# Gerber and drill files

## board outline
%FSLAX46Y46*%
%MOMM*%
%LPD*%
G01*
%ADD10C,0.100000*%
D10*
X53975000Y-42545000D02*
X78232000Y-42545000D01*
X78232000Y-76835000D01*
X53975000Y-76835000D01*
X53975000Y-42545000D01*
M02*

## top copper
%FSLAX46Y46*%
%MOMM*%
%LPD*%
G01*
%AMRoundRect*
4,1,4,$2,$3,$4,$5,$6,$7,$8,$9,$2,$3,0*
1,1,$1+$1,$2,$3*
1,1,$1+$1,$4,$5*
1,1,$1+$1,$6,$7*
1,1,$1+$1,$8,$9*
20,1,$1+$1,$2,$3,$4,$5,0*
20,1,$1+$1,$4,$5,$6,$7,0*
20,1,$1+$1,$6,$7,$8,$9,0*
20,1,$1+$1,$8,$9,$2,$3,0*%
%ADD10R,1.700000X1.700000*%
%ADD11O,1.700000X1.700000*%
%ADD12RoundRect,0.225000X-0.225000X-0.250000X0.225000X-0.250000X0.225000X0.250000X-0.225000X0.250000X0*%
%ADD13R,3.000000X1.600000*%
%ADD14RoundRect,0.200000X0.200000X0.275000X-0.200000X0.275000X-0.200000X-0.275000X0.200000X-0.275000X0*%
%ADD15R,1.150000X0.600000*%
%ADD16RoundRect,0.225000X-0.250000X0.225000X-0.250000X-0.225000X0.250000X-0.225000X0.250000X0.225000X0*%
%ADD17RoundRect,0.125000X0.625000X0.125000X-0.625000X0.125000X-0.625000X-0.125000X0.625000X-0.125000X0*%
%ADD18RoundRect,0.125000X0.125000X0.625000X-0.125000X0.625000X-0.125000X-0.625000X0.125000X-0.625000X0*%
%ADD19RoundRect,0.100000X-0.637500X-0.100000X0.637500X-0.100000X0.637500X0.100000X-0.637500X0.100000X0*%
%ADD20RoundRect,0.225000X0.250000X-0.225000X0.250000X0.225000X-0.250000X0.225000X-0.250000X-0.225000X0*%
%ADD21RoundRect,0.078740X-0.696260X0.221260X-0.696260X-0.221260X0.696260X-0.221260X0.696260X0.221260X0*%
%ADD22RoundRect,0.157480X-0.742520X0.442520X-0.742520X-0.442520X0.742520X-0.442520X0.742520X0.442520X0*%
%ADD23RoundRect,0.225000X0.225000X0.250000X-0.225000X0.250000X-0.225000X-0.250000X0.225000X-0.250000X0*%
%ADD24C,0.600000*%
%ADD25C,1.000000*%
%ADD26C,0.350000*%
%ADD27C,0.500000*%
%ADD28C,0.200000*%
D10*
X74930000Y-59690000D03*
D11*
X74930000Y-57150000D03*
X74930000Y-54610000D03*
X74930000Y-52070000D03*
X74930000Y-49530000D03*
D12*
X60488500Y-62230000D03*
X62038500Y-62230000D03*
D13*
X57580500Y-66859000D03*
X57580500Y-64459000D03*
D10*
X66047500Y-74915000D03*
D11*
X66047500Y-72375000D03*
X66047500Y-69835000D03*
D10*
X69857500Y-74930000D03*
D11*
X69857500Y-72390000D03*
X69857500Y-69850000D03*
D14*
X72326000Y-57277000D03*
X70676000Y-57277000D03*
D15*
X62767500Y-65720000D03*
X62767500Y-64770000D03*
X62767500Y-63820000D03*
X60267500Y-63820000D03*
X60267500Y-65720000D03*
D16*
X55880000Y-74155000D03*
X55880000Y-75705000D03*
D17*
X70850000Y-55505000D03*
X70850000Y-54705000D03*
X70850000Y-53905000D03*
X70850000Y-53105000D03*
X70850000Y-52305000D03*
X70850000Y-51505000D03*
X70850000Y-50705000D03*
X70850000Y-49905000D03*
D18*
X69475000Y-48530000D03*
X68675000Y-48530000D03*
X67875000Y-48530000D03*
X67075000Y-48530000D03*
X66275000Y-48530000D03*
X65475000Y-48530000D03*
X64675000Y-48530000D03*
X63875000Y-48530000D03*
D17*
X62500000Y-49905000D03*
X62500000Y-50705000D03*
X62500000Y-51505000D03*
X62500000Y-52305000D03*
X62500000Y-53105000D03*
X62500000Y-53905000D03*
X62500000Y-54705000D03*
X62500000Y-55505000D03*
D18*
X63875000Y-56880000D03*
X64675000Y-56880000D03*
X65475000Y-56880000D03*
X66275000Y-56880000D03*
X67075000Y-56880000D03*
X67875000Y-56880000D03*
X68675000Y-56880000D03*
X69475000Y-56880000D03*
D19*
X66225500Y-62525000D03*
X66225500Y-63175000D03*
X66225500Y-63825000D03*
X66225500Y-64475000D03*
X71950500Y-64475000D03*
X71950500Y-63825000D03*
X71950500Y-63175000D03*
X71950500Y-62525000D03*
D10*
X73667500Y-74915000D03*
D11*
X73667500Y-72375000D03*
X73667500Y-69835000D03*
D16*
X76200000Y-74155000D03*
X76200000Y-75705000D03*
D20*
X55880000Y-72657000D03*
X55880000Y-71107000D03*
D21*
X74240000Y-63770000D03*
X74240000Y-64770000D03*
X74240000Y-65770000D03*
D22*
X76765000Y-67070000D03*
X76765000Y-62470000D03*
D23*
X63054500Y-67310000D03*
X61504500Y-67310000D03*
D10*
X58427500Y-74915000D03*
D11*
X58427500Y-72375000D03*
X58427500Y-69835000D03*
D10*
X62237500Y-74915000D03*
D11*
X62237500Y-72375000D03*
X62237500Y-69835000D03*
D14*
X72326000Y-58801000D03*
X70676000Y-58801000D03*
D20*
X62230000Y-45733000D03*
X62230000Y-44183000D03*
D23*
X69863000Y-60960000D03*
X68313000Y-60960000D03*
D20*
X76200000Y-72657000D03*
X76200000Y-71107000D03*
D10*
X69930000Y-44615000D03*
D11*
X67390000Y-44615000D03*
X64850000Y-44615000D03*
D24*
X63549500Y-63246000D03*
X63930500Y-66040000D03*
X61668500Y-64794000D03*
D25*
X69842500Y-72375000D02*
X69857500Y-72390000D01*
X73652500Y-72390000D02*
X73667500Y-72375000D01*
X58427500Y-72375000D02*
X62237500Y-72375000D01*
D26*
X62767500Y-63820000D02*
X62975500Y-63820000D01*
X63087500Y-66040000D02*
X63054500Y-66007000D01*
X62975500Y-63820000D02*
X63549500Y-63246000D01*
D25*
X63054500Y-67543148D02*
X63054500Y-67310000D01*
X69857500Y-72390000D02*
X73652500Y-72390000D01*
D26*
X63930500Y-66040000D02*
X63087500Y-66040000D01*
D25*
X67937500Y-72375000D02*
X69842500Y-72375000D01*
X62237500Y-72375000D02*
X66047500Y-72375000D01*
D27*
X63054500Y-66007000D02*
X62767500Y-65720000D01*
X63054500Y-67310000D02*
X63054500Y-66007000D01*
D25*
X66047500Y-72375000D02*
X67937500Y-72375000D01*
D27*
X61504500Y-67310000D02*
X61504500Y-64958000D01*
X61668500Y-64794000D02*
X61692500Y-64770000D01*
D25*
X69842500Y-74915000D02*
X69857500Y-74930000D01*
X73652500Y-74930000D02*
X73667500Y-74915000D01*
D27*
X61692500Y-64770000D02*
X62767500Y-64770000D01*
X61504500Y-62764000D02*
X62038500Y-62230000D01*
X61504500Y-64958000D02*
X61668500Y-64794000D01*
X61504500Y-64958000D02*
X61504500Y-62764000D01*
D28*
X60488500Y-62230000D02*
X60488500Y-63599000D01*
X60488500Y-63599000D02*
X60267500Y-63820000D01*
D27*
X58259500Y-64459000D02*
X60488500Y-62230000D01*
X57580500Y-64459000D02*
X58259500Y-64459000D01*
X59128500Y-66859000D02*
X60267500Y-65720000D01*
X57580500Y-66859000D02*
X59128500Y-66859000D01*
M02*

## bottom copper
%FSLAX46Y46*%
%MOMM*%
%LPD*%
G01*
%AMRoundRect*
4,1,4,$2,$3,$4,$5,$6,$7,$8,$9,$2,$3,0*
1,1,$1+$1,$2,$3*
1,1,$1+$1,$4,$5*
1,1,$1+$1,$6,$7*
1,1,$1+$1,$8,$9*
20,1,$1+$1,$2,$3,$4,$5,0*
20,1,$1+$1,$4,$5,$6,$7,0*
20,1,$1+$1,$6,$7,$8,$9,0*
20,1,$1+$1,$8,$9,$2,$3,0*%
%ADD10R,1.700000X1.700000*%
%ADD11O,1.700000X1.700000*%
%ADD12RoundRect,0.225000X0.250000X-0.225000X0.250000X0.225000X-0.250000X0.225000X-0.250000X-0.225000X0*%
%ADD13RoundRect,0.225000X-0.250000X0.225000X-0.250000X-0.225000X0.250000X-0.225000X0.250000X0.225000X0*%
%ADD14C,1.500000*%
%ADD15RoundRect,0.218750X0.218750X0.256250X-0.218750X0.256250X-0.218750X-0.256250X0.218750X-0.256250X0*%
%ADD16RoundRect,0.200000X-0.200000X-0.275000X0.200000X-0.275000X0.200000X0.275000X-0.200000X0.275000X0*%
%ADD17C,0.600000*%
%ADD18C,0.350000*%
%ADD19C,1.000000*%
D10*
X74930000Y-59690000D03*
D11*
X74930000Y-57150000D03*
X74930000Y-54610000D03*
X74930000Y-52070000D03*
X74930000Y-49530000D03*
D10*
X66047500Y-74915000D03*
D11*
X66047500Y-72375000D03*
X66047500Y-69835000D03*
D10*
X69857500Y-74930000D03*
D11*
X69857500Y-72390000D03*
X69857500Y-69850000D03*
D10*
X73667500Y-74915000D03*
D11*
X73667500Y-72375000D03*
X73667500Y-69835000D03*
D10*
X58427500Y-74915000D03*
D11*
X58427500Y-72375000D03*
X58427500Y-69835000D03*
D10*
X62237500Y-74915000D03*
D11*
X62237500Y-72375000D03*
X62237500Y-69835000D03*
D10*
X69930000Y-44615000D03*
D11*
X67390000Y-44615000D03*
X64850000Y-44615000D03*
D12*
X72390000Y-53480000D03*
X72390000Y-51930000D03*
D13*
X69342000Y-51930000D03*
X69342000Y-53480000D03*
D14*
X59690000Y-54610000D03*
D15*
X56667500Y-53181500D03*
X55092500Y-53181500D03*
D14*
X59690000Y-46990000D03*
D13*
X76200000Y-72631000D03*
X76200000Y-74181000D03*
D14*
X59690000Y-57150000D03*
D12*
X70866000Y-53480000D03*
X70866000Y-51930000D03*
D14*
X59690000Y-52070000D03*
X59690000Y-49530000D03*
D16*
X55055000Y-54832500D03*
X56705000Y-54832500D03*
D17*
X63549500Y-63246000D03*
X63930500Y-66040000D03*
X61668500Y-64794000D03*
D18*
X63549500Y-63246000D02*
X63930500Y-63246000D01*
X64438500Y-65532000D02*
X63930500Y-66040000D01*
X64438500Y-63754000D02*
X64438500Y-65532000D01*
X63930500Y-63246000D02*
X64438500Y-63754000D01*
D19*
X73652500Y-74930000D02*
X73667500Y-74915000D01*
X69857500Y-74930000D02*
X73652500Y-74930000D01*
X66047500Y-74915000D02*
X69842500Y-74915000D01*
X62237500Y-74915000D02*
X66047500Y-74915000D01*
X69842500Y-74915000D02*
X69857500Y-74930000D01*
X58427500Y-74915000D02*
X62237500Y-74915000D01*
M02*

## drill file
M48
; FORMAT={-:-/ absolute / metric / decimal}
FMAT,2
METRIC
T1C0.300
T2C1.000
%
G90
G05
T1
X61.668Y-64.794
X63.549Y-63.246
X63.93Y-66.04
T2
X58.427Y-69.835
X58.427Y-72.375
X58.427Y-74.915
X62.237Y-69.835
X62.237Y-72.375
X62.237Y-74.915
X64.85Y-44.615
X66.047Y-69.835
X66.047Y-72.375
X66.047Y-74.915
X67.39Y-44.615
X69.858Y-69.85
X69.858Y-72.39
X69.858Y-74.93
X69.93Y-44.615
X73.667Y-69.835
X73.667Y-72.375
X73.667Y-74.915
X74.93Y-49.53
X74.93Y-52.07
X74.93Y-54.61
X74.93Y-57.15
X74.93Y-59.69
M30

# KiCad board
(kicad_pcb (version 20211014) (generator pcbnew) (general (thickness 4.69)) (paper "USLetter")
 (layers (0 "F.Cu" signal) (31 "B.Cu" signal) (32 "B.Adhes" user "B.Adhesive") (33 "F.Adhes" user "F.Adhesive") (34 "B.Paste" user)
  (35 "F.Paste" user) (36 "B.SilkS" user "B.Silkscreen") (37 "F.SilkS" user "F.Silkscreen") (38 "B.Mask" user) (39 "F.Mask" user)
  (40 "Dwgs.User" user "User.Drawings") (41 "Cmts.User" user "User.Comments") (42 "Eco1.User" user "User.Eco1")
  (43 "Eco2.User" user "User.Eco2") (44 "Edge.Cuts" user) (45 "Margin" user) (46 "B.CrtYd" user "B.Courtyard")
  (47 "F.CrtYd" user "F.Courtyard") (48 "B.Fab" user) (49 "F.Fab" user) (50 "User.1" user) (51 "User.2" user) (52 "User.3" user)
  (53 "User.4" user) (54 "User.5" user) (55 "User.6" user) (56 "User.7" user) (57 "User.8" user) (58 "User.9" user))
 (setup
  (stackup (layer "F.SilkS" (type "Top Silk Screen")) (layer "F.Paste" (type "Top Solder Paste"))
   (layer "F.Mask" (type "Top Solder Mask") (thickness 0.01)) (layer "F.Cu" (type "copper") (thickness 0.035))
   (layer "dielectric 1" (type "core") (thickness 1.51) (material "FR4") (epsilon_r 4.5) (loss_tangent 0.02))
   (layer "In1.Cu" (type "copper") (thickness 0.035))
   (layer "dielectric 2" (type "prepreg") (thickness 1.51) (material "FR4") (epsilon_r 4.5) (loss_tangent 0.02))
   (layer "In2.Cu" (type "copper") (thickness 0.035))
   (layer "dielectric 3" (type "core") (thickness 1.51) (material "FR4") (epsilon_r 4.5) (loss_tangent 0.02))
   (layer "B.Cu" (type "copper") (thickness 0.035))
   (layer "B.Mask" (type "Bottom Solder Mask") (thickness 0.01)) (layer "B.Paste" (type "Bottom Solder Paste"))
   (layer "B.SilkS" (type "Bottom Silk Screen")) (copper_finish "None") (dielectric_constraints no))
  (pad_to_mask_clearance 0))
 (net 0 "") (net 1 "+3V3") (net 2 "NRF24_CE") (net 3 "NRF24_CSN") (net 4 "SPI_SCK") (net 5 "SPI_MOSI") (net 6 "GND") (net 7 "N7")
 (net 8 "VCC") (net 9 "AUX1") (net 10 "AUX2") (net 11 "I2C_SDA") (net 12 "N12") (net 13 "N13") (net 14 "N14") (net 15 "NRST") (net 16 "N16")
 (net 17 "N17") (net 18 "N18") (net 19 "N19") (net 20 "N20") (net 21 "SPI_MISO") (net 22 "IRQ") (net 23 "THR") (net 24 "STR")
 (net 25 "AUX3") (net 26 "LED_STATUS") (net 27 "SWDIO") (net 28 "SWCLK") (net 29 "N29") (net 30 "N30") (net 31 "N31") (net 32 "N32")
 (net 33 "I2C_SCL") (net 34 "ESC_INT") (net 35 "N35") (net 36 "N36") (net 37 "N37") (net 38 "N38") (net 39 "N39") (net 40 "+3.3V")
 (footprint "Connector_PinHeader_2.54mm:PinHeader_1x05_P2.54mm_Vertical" (layer "F.Cu") (at 74.93 59.69 180)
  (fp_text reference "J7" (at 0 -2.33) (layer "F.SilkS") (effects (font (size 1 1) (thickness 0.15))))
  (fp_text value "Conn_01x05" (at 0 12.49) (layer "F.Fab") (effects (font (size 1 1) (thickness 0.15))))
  (pad "1" thru_hole rect (at 0 0 180) (size 1.7 1.7) (drill 1) (layers *.Cu *.Mask) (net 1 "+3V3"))
  (pad "2" thru_hole oval (at 0 2.54 180) (size 1.7 1.7) (drill 1) (layers *.Cu *.Mask) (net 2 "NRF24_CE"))
  (pad "3" thru_hole oval (at 0 5.08 180) (size 1.7 1.7) (drill 1) (layers *.Cu *.Mask) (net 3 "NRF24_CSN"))
  (pad "4" thru_hole oval (at 0 7.62 180) (size 1.7 1.7) (drill 1) (layers *.Cu *.Mask) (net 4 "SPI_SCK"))
  (pad "5" thru_hole oval (at 0 10.16 180) (size 1.7 1.7) (drill 1) (layers *.Cu *.Mask) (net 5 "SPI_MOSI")))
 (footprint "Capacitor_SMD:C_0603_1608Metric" (layer "F.Cu") (at 61.2635 62.23)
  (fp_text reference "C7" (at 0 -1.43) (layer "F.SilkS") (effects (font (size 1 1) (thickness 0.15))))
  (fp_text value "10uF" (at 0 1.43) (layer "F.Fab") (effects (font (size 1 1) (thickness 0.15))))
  (pad "1" smd roundrect (at -0.775 0) (size 0.9 0.95) (layers "F.Cu" "F.Paste" "F.Mask") (roundrect_rratio 0.25) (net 1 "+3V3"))
  (pad "2" smd roundrect (at 0.775 0) (size 0.9 0.95) (layers "F.Cu" "F.Paste" "F.Mask") (roundrect_rratio 0.25) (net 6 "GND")))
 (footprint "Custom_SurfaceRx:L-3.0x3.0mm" (layer "F.Cu") (at 57.5805 65.659 90)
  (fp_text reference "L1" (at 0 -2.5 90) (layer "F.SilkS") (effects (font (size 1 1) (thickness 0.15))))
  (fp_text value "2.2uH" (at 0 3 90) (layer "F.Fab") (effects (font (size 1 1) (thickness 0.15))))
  (pad "1" smd rect (at -1.2 0 90) (size 1.6 3) (layers "F.Cu" "F.Paste" "F.Mask") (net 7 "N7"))
  (pad "2" smd rect (at 1.2 0 90) (size 1.6 3) (layers "F.Cu" "F.Paste" "F.Mask") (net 1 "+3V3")))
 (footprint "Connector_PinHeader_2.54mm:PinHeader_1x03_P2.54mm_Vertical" (layer "F.Cu") (at 66.0475 74.915 180)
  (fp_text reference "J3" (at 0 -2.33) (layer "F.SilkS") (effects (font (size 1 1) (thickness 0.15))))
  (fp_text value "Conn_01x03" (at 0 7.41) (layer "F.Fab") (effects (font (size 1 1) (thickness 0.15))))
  (pad "1" thru_hole rect (at 0 0 180) (size 1.7 1.7) (drill 1) (layers *.Cu *.Mask) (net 6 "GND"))
  (pad "2" thru_hole oval (at 0 2.54 180) (size 1.7 1.7) (drill 1) (layers *.Cu *.Mask) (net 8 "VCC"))
  (pad "3" thru_hole oval (at 0 5.08 180) (size 1.7 1.7) (drill 1) (layers *.Cu *.Mask) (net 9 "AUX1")))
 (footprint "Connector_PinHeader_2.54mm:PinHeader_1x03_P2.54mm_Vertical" (layer "F.Cu") (at 69.8575 74.93 180)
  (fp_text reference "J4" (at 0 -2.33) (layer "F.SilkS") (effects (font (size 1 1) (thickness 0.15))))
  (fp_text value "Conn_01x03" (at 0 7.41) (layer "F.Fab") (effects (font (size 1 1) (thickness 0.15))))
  (pad "1" thru_hole rect (at 0 0 180) (size 1.7 1.7) (drill 1) (layers *.Cu *.Mask) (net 6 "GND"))
  (pad "2" thru_hole oval (at 0 2.54 180) (size 1.7 1.7) (drill 1) (layers *.Cu *.Mask) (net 8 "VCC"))
  (pad "3" thru_hole oval (at 0 5.08 180) (size 1.7 1.7) (drill 1) (layers *.Cu *.Mask) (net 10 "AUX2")))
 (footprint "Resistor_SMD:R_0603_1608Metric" (layer "F.Cu") (at 71.501 57.277 180)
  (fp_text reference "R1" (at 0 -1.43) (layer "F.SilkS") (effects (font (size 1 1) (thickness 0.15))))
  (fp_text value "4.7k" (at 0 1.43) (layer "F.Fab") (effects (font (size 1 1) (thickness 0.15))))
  (pad "1" smd roundrect (at -0.825 0 180) (size 0.8 0.95) (layers "F.Cu" "F.Paste" "F.Mask") (roundrect_rratio 0.25) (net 1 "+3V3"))
  (pad "2" smd roundrect (at 0.825 0 180) (size 0.8 0.95) (layers "F.Cu" "F.Paste" "F.Mask") (roundrect_rratio 0.25) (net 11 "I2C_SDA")))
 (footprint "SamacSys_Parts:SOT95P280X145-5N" (layer "F.Cu") (at 61.5175 64.77 180)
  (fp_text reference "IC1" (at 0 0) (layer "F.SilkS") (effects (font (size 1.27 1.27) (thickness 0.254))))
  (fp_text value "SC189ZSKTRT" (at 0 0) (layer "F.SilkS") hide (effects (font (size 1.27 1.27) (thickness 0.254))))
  (pad "1" smd rect locked (at -1.25 -0.95 270) (size 0.6 1.15) (layers "F.Cu" "F.Paste" "F.Mask") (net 8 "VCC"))
  (pad "2" smd rect locked (at -1.25 0 270) (size 0.6 1.15) (layers "F.Cu" "F.Paste" "F.Mask") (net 6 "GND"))
  (pad "3" smd rect locked (at -1.25 0.95 270) (size 0.6 1.15) (layers "F.Cu" "F.Paste" "F.Mask") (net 8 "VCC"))
  (pad "4" smd rect locked (at 1.25 0.95 270) (size 0.6 1.15) (layers "F.Cu" "F.Paste" "F.Mask") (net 1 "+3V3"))
  (pad "5" smd rect locked (at 1.25 -0.95 270) (size 0.6 1.15) (layers "F.Cu" "F.Paste" "F.Mask") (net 7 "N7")))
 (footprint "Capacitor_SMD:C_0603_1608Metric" (layer "F.Cu") (at 55.88 74.93 -90)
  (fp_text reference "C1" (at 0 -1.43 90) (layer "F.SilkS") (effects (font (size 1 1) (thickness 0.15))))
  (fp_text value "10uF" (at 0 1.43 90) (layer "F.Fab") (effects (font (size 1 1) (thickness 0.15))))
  (pad "1" smd roundrect (at -0.775 0 270) (size 0.9 0.95) (layers "F.Cu" "F.Paste" "F.Mask") (roundrect_rratio 0.25) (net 8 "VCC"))
  (pad "2" smd roundrect (at 0.775 0 270) (size 0.9 0.95) (layers "F.Cu" "F.Paste" "F.Mask") (roundrect_rratio 0.25) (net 6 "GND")))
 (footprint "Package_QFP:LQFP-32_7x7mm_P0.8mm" (layer "F.Cu") (at 66.675 52.705 180)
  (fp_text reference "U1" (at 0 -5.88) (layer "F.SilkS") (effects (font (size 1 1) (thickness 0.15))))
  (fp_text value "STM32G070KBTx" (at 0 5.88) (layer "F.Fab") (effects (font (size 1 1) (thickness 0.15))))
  (pad "1" smd roundrect (at -4.175 -2.8 180) (size 1.5 0.5) (layers "F.Cu" "F.Paste" "F.Mask") (roundrect_rratio 0.25) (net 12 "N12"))
  (pad "2" smd roundrect (at -4.175 -2 180) (size 1.5 0.5) (layers "F.Cu" "F.Paste" "F.Mask") (roundrect_rratio 0.25) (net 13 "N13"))
  (pad "3" smd roundrect (at -4.175 -1.2 180) (size 1.5 0.5) (layers "F.Cu" "F.Paste" "F.Mask") (roundrect_rratio 0.25) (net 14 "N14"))
  (pad "4" smd roundrect (at -4.175 -0.4 180) (size 1.5 0.5) (layers "F.Cu" "F.Paste" "F.Mask") (roundrect_rratio 0.25) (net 1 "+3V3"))
  (pad "5" smd roundrect (at -4.175 0.4 180) (size 1.5 0.5) (layers "F.Cu" "F.Paste" "F.Mask") (roundrect_rratio 0.25) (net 6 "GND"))
  (pad "6" smd roundrect (at -4.175 1.2 180) (size 1.5 0.5) (layers "F.Cu" "F.Paste" "F.Mask") (roundrect_rratio 0.25) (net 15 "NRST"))
  (pad "7" smd roundrect (at -4.175 2 180) (size 1.5 0.5) (layers "F.Cu" "F.Paste" "F.Mask") (roundrect_rratio 0.25) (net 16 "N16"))
  (pad "8" smd roundrect (at -4.175 2.8 180) (size 1.5 0.5) (layers "F.Cu" "F.Paste" "F.Mask") (roundrect_rratio 0.25) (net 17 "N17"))
  (pad "9" smd roundrect (at -2.8 4.175 180) (size 0.5 1.5) (layers "F.Cu" "F.Paste" "F.Mask") (roundrect_rratio 0.25) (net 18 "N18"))
  (pad "10" smd roundrect (at -2 4.175 180) (size 0.5 1.5) (layers "F.Cu" "F.Paste" "F.Mask") (roundrect_rratio 0.25) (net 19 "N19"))
  (pad "11" smd roundrect (at -1.2 4.175 180) (size 0.5 1.5) (layers "F.Cu" "F.Paste" "F.Mask") (roundrect_rratio 0.25) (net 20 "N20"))
  (pad "12" smd roundrect (at -0.4 4.175 180) (size 0.5 1.5) (layers "F.Cu" "F.Paste" "F.Mask") (roundrect_rratio 0.25) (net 4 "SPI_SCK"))
  (pad "13" smd roundrect (at 0.4 4.175 180) (size 0.5 1.5) (layers "F.Cu" "F.Paste" "F.Mask") (roundrect_rratio 0.25) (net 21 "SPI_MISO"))
  (pad "14" smd roundrect (at 1.2 4.175 180) (size 0.5 1.5) (layers "F.Cu" "F.Paste" "F.Mask") (roundrect_rratio 0.25) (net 5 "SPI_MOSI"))
  (pad "15" smd roundrect (at 2 4.175 180) (size 0.5 1.5) (layers "F.Cu" "F.Paste" "F.Mask") (roundrect_rratio 0.25) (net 3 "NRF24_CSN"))
  (pad "16" smd roundrect (at 2.8 4.175 180) (size 0.5 1.5) (layers "F.Cu" "F.Paste" "F.Mask") (roundrect_rratio 0.25) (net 2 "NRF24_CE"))
  (pad "17" smd roundrect (at 4.175 2.8 180) (size 1.5 0.5) (layers "F.Cu" "F.Paste" "F.Mask") (roundrect_rratio 0.25) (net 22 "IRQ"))
  (pad "18" smd roundrect (at 4.175 2 180) (size 1.5 0.5) (layers "F.Cu" "F.Paste" "F.Mask") (roundrect_rratio 0.25) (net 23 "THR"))
  (pad "19" smd roundrect (at 4.175 1.2 180) (size 1.5 0.5) (layers "F.Cu" "F.Paste" "F.Mask") (roundrect_rratio 0.25) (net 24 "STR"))
  (pad "20" smd roundrect (at 4.175 0.4 180) (size 1.5 0.5) (layers "F.Cu" "F.Paste" "F.Mask") (roundrect_rratio 0.25) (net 9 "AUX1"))
  (pad "21" smd roundrect (at 4.175 -0.4 180) (size 1.5 0.5) (layers "F.Cu" "F.Paste" "F.Mask") (roundrect_rratio 0.25) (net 10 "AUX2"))
  (pad "22" smd roundrect (at 4.175 -1.2 180) (size 1.5 0.5) (layers "F.Cu" "F.Paste" "F.Mask") (roundrect_rratio 0.25) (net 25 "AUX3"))
  (pad "23" smd roundrect (at 4.175 -2 180) (size 1.5 0.5) (layers "F.Cu" "F.Paste" "F.Mask") (roundrect_rratio 0.25) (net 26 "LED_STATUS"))
  (pad "24" smd roundrect (at 4.175 -2.8 180) (size 1.5 0.5) (layers "F.Cu" "F.Paste" "F.Mask") (roundrect_rratio 0.25) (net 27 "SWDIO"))
  (pad "25" smd roundrect (at 2.8 -4.175 180) (size 0.5 1.5) (layers "F.Cu" "F.Paste" "F.Mask") (roundrect_rratio 0.25) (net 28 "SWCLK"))
  (pad "26" smd roundrect (at 2 -4.175 180) (size 0.5 1.5) (layers "F.Cu" "F.Paste" "F.Mask") (roundrect_rratio 0.25) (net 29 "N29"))
  (pad "27" smd roundrect (at 1.2 -4.175 180) (size 0.5 1.5) (layers "F.Cu" "F.Paste" "F.Mask") (roundrect_rratio 0.25) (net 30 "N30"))
  (pad "28" smd roundrect (at 0.4 -4.175 180) (size 0.5 1.5) (layers "F.Cu" "F.Paste" "F.Mask") (roundrect_rratio 0.25) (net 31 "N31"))
  (pad "29" smd roundrect (at -0.4 -4.175 180) (size 0.5 1.5) (layers "F.Cu" "F.Paste" "F.Mask") (roundrect_rratio 0.25) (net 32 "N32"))
  (pad "30" smd roundrect (at -1.2 -4.175 180) (size 0.5 1.5) (layers "F.Cu" "F.Paste" "F.Mask") (roundrect_rratio 0.25) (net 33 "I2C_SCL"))
  (pad "31" smd roundrect (at -2 -4.175 180) (size 0.5 1.5) (layers "F.Cu" "F.Paste" "F.Mask") (roundrect_rratio 0.25) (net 11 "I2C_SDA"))
  (pad "32" smd roundrect (at -2.8 -4.175 180) (size 0.5 1.5) (layers "F.Cu" "F.Paste" "F.Mask") (roundrect_rratio 0.25) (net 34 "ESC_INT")))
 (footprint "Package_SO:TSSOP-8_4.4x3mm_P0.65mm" (layer "F.Cu") (at 69.088 63.5)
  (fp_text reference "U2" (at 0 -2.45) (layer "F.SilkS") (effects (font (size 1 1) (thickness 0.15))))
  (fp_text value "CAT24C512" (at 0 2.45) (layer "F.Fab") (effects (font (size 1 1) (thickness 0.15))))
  (pad "1" smd roundrect (at -2.8625 -0.975) (size 1.475 0.4) (layers "F.Cu" "F.Paste" "F.Mask") (roundrect_rratio 0.25) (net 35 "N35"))
  (pad "2" smd roundrect (at -2.8625 -0.325) (size 1.475 0.4) (layers "F.Cu" "F.Paste" "F.Mask") (roundrect_rratio 0.25) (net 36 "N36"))
  (pad "3" smd roundrect (at -2.8625 0.325) (size 1.475 0.4) (layers "F.Cu" "F.Paste" "F.Mask") (roundrect_rratio 0.25) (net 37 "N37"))
  (pad "4" smd roundrect (at -2.8625 0.975) (size 1.475 0.4) (layers "F.Cu" "F.Paste" "F.Mask") (roundrect_rratio 0.25) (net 6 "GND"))
  (pad "5" smd roundrect (at 2.8625 0.975) (size 1.475 0.4) (layers "F.Cu" "F.Paste" "F.Mask") (roundrect_rratio 0.25) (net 11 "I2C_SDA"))
  (pad "6" smd roundrect (at 2.8625 0.325) (size 1.475 0.4) (layers "F.Cu" "F.Paste" "F.Mask") (roundrect_rratio 0.25) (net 33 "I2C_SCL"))
  (pad "7" smd roundrect (at 2.8625 -0.325) (size 1.475 0.4) (layers "F.Cu" "F.Paste" "F.Mask") (roundrect_rratio 0.25) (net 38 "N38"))
  (pad "8" smd roundrect (at 2.8625 -0.975) (size 1.475 0.4) (layers "F.Cu" "F.Paste" "F.Mask") (roundrect_rratio 0.25) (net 1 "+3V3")))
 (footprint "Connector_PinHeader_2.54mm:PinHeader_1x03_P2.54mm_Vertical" (layer "F.Cu") (at 73.6675 74.915 180)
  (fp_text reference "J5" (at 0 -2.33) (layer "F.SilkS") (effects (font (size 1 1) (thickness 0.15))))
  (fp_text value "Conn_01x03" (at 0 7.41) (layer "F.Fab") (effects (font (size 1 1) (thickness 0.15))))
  (pad "1" thru_hole rect (at 0 0 180) (size 1.7 1.7) (drill 1) (layers *.Cu *.Mask) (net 6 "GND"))
  (pad "2" thru_hole oval (at 0 2.54 180) (size 1.7 1.7) (drill 1) (layers *.Cu *.Mask) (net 8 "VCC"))
  (pad "3" thru_hole oval (at 0 5.08 180) (size 1.7 1.7) (drill 1) (layers *.Cu *.Mask) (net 25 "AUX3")))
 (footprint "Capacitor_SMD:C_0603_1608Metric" (layer "F.Cu") (at 76.2 74.93 -90)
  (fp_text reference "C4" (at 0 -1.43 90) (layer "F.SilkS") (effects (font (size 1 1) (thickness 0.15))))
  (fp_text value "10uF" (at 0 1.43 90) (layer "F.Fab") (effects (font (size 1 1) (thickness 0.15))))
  (pad "1" smd roundrect (at -0.775 0 270) (size 0.9 0.95) (layers "F.Cu" "F.Paste" "F.Mask") (roundrect_rratio 0.25) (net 8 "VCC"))
  (pad "2" smd roundrect (at 0.775 0 270) (size 0.9 0.95) (layers "F.Cu" "F.Paste" "F.Mask") (roundrect_rratio 0.25) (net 6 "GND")))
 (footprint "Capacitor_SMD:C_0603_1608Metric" (layer "F.Cu") (at 55.88 71.882 90)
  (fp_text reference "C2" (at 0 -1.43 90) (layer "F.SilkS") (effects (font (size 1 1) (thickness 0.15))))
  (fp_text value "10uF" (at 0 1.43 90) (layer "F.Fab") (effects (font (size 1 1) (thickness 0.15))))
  (pad "1" smd roundrect (at -0.775 0 90) (size 0.9 0.95) (layers "F.Cu" "F.Paste" "F.Mask") (roundrect_rratio 0.25) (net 8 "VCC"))
  (pad "2" smd roundrect (at 0.775 0 90) (size 0.9 0.95) (layers "F.Cu" "F.Paste" "F.Mask") (roundrect_rratio 0.25) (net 6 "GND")))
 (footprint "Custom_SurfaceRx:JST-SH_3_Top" (layer "F.Cu") (at 74.24 64.77 -90)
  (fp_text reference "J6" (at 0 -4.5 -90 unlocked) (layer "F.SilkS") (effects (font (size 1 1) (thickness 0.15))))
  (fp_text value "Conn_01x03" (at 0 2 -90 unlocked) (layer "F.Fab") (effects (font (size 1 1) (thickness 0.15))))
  (pad "1" smd roundrect (at -1 0 270) (size 0.6 1.55) (layers "F.Cu" "F.Paste" "F.Mask") (roundrect_rratio 0.1312335958) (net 34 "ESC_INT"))
  (pad "2" smd roundrect (at 0 0 270) (size 0.6 1.55) (layers "F.Cu" "F.Paste" "F.Mask") (roundrect_rratio 0.1312335958) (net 11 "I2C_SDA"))
  (pad "3" smd roundrect (at 1 0 270) (size 0.6 1.55) (layers "F.Cu" "F.Paste" "F.Mask") (roundrect_rratio 0.1312335958) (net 33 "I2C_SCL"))
  (pad "MP" smd roundrect (at 2.3 -2.525 270) (size 1.2 1.8) (layers "F.Cu" "F.Paste" "F.Mask") (roundrect_rratio 0.1312335958))
  (pad "MP" smd roundrect (at -2.3 -2.525 270) (size 1.2 1.8) (layers "F.Cu" "F.Paste" "F.Mask") (roundrect_rratio 0.1312335958)))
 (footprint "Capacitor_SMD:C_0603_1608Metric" (layer "F.Cu") (at 62.2795 67.31 180)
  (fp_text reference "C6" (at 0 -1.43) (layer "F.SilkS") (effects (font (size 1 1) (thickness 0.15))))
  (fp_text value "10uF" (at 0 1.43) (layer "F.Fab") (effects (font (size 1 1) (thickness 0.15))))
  (pad "1" smd roundrect (at -0.775 0 180) (size 0.9 0.95) (layers "F.Cu" "F.Paste" "F.Mask") (roundrect_rratio 0.25) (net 8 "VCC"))
  (pad "2" smd roundrect (at 0.775 0 180) (size 0.9 0.95) (layers "F.Cu" "F.Paste" "F.Mask") (roundrect_rratio 0.25) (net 6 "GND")))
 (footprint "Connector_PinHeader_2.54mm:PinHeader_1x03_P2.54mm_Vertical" (layer "F.Cu") (at 58.4275 74.915 180)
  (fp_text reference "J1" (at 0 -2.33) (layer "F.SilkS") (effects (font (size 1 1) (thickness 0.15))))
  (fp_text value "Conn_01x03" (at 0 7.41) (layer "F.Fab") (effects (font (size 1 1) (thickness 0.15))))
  (pad "1" thru_hole rect (at 0 0 180) (size 1.7 1.7) (drill 1) (layers *.Cu *.Mask) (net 6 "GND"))
  (pad "2" thru_hole oval (at 0 2.54 180) (size 1.7 1.7) (drill 1) (layers *.Cu *.Mask) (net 8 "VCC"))
  (pad "3" thru_hole oval (at 0 5.08 180) (size 1.7 1.7) (drill 1) (layers *.Cu *.Mask) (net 23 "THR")))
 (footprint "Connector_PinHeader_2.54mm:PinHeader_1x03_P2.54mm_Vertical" (layer "F.Cu") (at 62.2375 74.915 180)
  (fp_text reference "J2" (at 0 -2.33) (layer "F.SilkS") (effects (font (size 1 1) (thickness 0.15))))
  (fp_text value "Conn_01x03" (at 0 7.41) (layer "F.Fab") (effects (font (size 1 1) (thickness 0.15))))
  (pad "1" thru_hole rect (at 0 0 180) (size 1.7 1.7) (drill 1) (layers *.Cu *.Mask) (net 6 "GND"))
  (pad "2" thru_hole oval (at 0 2.54 180) (size 1.7 1.7) (drill 1) (layers *.Cu *.Mask) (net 8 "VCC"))
  (pad "3" thru_hole oval (at 0 5.08 180) (size 1.7 1.7) (drill 1) (layers *.Cu *.Mask) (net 24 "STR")))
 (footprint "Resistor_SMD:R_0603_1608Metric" (layer "F.Cu") (at 71.501 58.801 180)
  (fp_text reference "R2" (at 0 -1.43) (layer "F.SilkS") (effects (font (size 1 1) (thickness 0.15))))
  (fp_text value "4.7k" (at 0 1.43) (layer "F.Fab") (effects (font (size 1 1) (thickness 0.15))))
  (pad "1" smd roundrect (at -0.825 0 180) (size 0.8 0.95) (layers "F.Cu" "F.Paste" "F.Mask") (roundrect_rratio 0.25) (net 1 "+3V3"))
  (pad "2" smd roundrect (at 0.825 0 180) (size 0.8 0.95) (layers "F.Cu" "F.Paste" "F.Mask") (roundrect_rratio 0.25) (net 33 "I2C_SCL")))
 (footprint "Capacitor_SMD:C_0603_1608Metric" (layer "F.Cu") (at 62.23 44.958 90)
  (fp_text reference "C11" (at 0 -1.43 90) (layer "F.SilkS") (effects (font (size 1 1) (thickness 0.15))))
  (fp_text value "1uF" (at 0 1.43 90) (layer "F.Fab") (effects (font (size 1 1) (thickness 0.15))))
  (pad "1" smd roundrect (at -0.775 0 90) (size 0.9 0.95) (layers "F.Cu" "F.Paste" "F.Mask") (roundrect_rratio 0.25) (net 1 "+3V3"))
  (pad "2" smd roundrect (at 0.775 0 90) (size 0.9 0.95) (layers "F.Cu" "F.Paste" "F.Mask") (roundrect_rratio 0.25) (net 6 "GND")))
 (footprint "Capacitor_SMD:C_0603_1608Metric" (layer "F.Cu") (at 69.088 60.96 180)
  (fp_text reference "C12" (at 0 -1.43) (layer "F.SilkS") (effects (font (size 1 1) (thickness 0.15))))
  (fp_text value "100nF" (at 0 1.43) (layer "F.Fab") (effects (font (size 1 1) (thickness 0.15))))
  (pad "1" smd roundrect (at -0.775 0 180) (size 0.9 0.95) (layers "F.Cu" "F.Paste" "F.Mask") (roundrect_rratio 0.25) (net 1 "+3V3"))
  (pad "2" smd roundrect (at 0.775 0 180) (size 0.9 0.95) (layers "F.Cu" "F.Paste" "F.Mask") (roundrect_rratio 0.25) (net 6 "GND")))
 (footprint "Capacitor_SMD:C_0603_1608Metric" (layer "F.Cu") (at 76.2 71.882 90)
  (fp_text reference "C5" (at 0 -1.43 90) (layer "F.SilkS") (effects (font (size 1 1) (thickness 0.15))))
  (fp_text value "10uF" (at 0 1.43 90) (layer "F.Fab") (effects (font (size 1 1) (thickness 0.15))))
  (pad "1" smd roundrect (at -0.775 0 90) (size 0.9 0.95) (layers "F.Cu" "F.Paste" "F.Mask") (roundrect_rratio 0.25) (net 8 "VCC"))
  (pad "2" smd roundrect (at 0.775 0 90) (size 0.9 0.95) (layers "F.Cu" "F.Paste" "F.Mask") (roundrect_rratio 0.25) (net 6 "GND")))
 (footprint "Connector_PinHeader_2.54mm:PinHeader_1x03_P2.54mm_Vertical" (layer "F.Cu") (at 69.93 44.615 -90)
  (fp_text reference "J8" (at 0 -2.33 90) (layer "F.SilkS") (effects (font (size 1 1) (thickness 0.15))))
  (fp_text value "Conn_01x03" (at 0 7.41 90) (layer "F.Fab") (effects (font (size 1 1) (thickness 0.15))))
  (pad "1" thru_hole rect (at 0 0 270) (size 1.7 1.7) (drill 1) (layers *.Cu *.Mask) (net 21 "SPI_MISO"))
  (pad "2" thru_hole oval (at 0 2.54 270) (size 1.7 1.7) (drill 1) (layers *.Cu *.Mask) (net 22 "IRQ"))
  (pad "3" thru_hole oval (at 0 5.08 270) (size 1.7 1.7) (drill 1) (layers *.Cu *.Mask) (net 6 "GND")))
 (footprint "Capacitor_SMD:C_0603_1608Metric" (layer "B.Cu") (at 72.39 52.705 90)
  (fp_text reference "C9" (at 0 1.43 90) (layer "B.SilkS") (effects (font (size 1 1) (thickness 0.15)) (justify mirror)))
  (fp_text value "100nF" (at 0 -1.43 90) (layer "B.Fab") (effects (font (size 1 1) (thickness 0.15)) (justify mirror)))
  (pad "1" smd roundrect (at -0.775 0 90) (size 0.9 0.95) (layers "B.Cu" "B.Paste" "B.Mask") (roundrect_rratio 0.25) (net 1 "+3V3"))
  (pad "2" smd roundrect (at 0.775 0 90) (size 0.9 0.95) (layers "B.Cu" "B.Paste" "B.Mask") (roundrect_rratio 0.25) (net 6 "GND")))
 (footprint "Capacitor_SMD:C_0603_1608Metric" (layer "B.Cu") (at 69.342 52.705 -90)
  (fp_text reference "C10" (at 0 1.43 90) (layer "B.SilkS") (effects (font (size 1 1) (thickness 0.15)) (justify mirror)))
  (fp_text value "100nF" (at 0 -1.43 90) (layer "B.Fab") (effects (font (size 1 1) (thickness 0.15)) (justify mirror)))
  (pad "1" smd roundrect (at -0.775 0 270) (size 0.9 0.95) (layers "B.Cu" "B.Paste" "B.Mask") (roundrect_rratio 0.25) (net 15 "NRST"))
  (pad "2" smd roundrect (at 0.775 0 270) (size 0.9 0.95) (layers "B.Cu" "B.Paste" "B.Mask") (roundrect_rratio 0.25) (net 6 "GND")))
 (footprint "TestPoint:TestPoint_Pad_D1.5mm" (layer "B.Cu") (at 59.69 54.61 180)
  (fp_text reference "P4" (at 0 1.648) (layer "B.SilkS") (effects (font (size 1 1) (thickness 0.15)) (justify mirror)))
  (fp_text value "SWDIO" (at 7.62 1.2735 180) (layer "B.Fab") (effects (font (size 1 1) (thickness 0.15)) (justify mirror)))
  (pad "1" smd circle (at 0 0 180) (size 1.5 1.5) (layers "B.Cu" "B.Mask") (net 27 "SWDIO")))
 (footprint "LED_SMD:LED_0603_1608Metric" (layer "B.Cu") (at 55.88 53.1815 180)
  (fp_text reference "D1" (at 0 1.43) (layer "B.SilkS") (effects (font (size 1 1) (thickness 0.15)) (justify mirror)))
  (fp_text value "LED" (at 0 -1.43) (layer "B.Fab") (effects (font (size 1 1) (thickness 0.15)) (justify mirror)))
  (pad "1" smd roundrect (at -0.7875 0 180) (size 0.875 0.95) (layers "B.Cu" "B.Paste" "B.Mask") (roundrect_rratio 0.25) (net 6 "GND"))
  (pad "2" smd roundrect (at 0.7875 0 180) (size 0.875 0.95) (layers "B.Cu" "B.Paste" "B.Mask") (roundrect_rratio 0.25) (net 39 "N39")))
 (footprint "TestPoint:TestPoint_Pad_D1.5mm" (layer "B.Cu") (at 59.69 46.99 180)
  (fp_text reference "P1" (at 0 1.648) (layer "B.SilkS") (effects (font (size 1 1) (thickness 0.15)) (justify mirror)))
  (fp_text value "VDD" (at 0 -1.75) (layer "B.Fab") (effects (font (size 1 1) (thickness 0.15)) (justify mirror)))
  (pad "1" smd circle (at 0 0 180) (size 1.5 1.5) (layers "B.Cu" "B.Mask") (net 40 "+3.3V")))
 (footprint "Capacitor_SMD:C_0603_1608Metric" (layer "B.Cu") (at 76.2 73.406 -90)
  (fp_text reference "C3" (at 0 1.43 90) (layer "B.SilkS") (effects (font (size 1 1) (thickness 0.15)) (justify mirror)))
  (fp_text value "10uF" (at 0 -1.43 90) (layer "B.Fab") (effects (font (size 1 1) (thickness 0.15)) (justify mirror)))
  (pad "1" smd roundrect (at -0.775 0 270) (size 0.9 0.95) (layers "B.Cu" "B.Paste" "B.Mask") (roundrect_rratio 0.25) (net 8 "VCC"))
  (pad "2" smd roundrect (at 0.775 0 270) (size 0.9 0.95) (layers "B.Cu" "B.Paste" "B.Mask") (roundrect_rratio 0.25) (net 6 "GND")))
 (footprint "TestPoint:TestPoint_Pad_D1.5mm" (layer "B.Cu") (at 59.69 57.15 180)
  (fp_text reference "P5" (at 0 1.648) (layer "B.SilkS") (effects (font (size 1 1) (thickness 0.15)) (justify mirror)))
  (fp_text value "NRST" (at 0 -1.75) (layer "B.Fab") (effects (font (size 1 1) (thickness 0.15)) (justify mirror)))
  (pad "1" smd circle (at 0 0 180) (size 1.5 1.5) (layers "B.Cu" "B.Mask") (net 15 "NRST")))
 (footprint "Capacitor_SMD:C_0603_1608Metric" (layer "B.Cu") (at 70.866 52.705 90)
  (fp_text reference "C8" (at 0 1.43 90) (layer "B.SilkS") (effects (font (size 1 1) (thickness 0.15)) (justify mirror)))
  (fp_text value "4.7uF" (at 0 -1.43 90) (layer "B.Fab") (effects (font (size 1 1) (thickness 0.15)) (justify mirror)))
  (pad "1" smd roundrect (at -0.775 0 90) (size 0.9 0.95) (layers "B.Cu" "B.Paste" "B.Mask") (roundrect_rratio 0.25) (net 1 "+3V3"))
  (pad "2" smd roundrect (at 0.775 0 90) (size 0.9 0.95) (layers "B.Cu" "B.Paste" "B.Mask") (roundrect_rratio 0.25) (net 6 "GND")))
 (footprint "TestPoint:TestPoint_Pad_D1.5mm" (layer "B.Cu") (at 59.69 52.07 180)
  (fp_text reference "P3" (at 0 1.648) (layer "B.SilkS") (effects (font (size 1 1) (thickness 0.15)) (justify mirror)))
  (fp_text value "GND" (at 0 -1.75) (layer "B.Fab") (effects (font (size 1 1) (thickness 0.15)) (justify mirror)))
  (pad "1" smd circle (at 0 0 180) (size 1.5 1.5) (layers "B.Cu" "B.Mask") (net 6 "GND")))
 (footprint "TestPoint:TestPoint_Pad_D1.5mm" (layer "B.Cu") (at 59.69 49.53 180)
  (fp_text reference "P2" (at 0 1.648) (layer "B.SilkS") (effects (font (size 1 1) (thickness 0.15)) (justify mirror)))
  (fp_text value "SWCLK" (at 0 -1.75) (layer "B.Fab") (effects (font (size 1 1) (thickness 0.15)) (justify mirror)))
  (pad "1" smd circle (at 0 0 180) (size 1.5 1.5) (layers "B.Cu" "B.Mask") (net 28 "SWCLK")))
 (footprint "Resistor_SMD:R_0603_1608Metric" (layer "B.Cu") (at 55.88 54.8325)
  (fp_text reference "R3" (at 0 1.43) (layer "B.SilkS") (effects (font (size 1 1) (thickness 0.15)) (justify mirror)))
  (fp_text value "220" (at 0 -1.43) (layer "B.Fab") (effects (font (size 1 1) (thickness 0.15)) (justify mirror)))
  (pad "1" smd roundrect (at -0.825 0) (size 0.8 0.95) (layers "B.Cu" "B.Paste" "B.Mask") (roundrect_rratio 0.25) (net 39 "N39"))
  (pad "2" smd roundrect (at 0.825 0) (size 0.8 0.95) (layers "B.Cu" "B.Paste" "B.Mask") (roundrect_rratio 0.25) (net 26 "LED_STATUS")))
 (gr_rect (start 53.975 42.545) (end 78.232 76.835) (layer "Edge.Cuts") (width 0.1) (fill none))
 (segment (start 69.8425 72.375) (end 69.8575 72.39) (width 1) (layer "F.Cu") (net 8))
 (segment (start 73.6525 72.39) (end 73.6675 72.375) (width 1) (layer "F.Cu") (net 8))
 (segment (start 58.4275 72.375) (end 62.2375 72.375) (width 1) (layer "F.Cu") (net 8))
 (segment (start 62.7675 63.82) (end 62.9755 63.82) (width 0.35) (layer "F.Cu") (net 8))
 (segment (start 63.0875 66.04) (end 63.0545 66.007) (width 0.35) (layer "F.Cu") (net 8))
 (segment (start 62.9755 63.82) (end 63.5495 63.246) (width 0.35) (layer "F.Cu") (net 8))
 (segment (start 63.0545 67.543148) (end 63.0545 67.31) (width 1) (layer "F.Cu") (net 8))
 (segment (start 69.8575 72.39) (end 73.6525 72.39) (width 1) (layer "F.Cu") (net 8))
 (segment (start 63.9305 66.04) (end 63.0875 66.04) (width 0.35) (layer "F.Cu") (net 8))
 (segment (start 67.9375 72.375) (end 69.8425 72.375) (width 1) (layer "F.Cu") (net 8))
 (segment (start 62.2375 72.375) (end 66.0475 72.375) (width 1) (layer "F.Cu") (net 8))
 (segment (start 63.0545 66.007) (end 62.7675 65.72) (width 0.5) (layer "F.Cu") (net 8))
 (segment (start 63.0545 67.31) (end 63.0545 66.007) (width 0.5) (layer "F.Cu") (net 8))
 (segment (start 66.0475 72.375) (end 67.9375 72.375) (width 1) (layer "F.Cu") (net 8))
 (via (at 63.5495 63.246) (size 0.6) (drill 0.3) (layers "F.Cu" "B.Cu") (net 8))
 (via (at 63.9305 66.04) (size 0.6) (drill 0.3) (layers "F.Cu" "B.Cu") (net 8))
 (segment (start 63.5495 63.246) (end 63.9305 63.246) (width 0.35) (layer "B.Cu") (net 8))
 (segment (start 64.4385 65.532) (end 63.9305 66.04) (width 0.35) (layer "B.Cu") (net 8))
 (segment (start 64.4385 63.754) (end 64.4385 65.532) (width 0.35) (layer "B.Cu") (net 8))
 (segment (start 63.9305 63.246) (end 64.4385 63.754) (width 0.35) (layer "B.Cu") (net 8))
 (segment (start 61.5045 67.31) (end 61.5045 64.958) (width 0.5) (layer "F.Cu") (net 6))
 (segment (start 61.6685 64.794) (end 61.6925 64.77) (width 0.5) (layer "F.Cu") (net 6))
 (segment (start 69.8425 74.915) (end 69.8575 74.93) (width 1) (layer "F.Cu") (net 6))
 (segment (start 73.6525 74.93) (end 73.6675 74.915) (width 1) (layer "F.Cu") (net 6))
 (segment (start 61.6925 64.77) (end 62.7675 64.77) (width 0.5) (layer "F.Cu") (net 6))
 (segment (start 61.5045 62.764) (end 62.0385 62.23) (width 0.5) (layer "F.Cu") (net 6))
 (segment (start 61.5045 64.958) (end 61.6685 64.794) (width 0.5) (layer "F.Cu") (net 6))
 (segment (start 61.5045 64.958) (end 61.5045 62.764) (width 0.5) (layer "F.Cu") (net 6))
 (via (at 61.6685 64.794) (size 0.6) (drill 0.3) (layers "F.Cu" "B.Cu") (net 6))
 (segment (start 73.6525 74.93) (end 73.6675 74.915) (width 1) (layer "B.Cu") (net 6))
 (segment (start 69.8575 74.93) (end 73.6525 74.93) (width 1) (layer "B.Cu") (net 6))
 (segment (start 66.0475 74.915) (end 69.8425 74.915) (width 1) (layer "B.Cu") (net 6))
 (segment (start 62.2375 74.915) (end 66.0475 74.915) (width 1) (layer "B.Cu") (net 6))
 (segment (start 69.8425 74.915) (end 69.8575 74.93) (width 1) (layer "B.Cu") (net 6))
 (segment (start 58.4275 74.915) (end 62.2375 74.915) (width 1) (layer "B.Cu") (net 6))
 (segment (start 60.4885 62.23) (end 60.4885 63.599) (width 0.2) (layer "F.Cu") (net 1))
 (segment (start 60.4885 63.599) (end 60.2675 63.82) (width 0.2) (layer "F.Cu") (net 1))
 (segment (start 58.2595 64.459) (end 60.4885 62.23) (width 0.5) (layer "F.Cu") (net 1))
 (segment (start 57.5805 64.459) (end 58.2595 64.459) (width 0.5) (layer "F.Cu") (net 1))
 (segment (start 59.1285 66.859) (end 60.2675 65.72) (width 0.5) (layer "F.Cu") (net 7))
 (segment (start 57.5805 66.859) (end 59.1285 66.859) (width 0.5) (layer "F.Cu") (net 7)))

